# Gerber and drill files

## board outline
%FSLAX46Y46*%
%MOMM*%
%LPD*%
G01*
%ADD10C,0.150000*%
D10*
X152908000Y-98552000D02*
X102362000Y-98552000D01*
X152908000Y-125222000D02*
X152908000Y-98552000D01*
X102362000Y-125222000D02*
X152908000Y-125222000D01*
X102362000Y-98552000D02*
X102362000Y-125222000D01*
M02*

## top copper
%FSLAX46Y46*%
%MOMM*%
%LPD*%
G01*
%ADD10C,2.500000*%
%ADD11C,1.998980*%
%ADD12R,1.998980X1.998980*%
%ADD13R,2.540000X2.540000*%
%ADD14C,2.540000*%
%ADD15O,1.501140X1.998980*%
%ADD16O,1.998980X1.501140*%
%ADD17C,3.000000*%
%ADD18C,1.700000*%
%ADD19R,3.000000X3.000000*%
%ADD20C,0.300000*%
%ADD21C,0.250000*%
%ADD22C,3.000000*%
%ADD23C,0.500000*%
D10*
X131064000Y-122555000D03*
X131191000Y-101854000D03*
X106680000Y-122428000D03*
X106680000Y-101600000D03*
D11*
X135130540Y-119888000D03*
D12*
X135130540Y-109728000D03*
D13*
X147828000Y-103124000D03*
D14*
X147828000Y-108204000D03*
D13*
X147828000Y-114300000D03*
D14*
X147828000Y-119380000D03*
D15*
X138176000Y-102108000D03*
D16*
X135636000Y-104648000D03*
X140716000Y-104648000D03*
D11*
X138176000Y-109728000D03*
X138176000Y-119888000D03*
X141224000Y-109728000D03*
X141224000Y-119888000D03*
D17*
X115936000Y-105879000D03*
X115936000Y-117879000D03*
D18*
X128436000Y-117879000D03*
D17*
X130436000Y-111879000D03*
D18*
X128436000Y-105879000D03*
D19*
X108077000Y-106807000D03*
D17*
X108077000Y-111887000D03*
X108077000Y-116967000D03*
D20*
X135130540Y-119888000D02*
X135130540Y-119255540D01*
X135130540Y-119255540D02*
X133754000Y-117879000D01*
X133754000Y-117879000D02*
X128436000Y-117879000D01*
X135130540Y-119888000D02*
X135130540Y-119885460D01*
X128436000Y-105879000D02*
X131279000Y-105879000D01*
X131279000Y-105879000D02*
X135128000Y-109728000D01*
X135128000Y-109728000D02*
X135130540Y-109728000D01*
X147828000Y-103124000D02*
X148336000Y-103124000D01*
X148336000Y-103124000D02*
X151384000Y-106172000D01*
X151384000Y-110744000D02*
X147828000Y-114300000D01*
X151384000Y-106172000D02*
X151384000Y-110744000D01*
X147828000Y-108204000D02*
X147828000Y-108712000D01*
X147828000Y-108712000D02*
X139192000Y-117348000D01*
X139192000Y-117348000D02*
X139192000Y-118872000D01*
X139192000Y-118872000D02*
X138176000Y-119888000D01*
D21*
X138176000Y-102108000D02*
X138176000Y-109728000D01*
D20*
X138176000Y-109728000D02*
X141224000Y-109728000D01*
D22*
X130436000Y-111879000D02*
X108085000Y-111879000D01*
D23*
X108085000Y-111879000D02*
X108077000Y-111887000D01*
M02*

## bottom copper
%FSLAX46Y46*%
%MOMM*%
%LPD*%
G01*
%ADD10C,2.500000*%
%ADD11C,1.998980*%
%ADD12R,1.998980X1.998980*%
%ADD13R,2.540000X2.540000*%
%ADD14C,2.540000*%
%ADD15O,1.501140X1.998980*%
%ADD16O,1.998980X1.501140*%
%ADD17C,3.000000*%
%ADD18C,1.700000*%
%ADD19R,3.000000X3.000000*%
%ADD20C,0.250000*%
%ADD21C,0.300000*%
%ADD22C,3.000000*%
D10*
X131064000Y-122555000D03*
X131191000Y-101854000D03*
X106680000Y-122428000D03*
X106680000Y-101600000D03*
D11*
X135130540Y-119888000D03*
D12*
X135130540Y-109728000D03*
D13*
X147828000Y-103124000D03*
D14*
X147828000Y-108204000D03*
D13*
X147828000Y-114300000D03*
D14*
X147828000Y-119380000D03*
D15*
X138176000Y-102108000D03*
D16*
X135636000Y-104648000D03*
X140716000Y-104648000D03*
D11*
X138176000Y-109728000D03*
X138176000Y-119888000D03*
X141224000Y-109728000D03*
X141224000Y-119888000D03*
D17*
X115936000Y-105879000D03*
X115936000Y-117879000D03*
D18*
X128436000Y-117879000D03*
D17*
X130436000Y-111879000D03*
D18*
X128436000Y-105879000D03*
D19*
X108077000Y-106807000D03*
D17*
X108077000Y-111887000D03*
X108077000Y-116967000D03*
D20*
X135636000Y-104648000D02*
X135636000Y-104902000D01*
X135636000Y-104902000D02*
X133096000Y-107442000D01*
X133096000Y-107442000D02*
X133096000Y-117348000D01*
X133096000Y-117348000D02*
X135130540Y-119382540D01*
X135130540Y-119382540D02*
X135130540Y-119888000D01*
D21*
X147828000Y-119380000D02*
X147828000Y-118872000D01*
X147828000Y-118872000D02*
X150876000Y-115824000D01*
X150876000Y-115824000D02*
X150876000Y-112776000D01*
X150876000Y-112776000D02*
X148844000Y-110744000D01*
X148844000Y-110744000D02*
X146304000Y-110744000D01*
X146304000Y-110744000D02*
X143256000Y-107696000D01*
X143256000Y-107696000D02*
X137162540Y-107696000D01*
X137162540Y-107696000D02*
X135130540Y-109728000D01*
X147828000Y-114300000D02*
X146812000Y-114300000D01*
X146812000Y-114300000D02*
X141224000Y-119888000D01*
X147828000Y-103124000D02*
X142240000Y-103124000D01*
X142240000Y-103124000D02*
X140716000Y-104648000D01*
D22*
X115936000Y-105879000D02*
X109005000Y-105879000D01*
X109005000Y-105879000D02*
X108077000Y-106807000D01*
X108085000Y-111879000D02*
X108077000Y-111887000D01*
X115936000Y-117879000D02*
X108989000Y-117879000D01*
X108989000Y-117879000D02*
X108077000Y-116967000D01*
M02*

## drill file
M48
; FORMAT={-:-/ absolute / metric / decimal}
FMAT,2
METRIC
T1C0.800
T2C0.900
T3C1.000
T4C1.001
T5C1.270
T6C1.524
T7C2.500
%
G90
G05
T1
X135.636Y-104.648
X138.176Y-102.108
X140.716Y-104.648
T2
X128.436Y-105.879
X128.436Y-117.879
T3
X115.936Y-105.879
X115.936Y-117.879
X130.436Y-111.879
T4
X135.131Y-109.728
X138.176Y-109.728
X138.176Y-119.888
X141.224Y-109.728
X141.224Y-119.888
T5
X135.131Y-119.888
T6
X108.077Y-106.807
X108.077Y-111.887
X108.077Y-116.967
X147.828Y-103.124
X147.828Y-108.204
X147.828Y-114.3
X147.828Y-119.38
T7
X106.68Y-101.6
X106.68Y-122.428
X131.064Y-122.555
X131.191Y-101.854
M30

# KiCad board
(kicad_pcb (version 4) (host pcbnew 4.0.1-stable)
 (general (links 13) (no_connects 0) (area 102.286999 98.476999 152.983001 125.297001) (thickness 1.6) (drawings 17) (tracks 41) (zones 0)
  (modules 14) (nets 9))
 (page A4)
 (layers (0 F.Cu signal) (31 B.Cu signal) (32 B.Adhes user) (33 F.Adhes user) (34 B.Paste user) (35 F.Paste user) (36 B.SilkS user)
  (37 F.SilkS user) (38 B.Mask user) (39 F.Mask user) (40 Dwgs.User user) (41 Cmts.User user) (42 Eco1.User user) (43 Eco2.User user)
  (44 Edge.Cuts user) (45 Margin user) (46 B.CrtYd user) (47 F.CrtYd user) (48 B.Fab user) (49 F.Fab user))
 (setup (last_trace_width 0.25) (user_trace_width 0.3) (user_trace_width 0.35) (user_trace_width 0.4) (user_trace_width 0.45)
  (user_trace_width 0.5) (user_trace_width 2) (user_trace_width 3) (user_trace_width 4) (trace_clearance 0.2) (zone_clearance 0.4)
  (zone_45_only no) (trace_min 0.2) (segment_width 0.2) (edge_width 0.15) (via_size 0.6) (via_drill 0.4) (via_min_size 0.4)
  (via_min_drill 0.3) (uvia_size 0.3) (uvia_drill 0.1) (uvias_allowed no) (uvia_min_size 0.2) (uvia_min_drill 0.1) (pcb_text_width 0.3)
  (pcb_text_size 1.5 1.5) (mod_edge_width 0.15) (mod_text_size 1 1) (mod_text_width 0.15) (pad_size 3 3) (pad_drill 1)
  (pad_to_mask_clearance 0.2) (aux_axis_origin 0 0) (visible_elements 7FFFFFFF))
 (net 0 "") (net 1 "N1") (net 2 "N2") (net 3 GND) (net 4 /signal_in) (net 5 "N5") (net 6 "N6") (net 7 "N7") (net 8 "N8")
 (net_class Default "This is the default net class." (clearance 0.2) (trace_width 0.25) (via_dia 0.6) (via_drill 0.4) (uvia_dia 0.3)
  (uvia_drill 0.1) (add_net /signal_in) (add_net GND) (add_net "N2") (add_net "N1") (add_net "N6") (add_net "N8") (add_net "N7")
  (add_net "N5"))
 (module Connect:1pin (layer F.Cu) (at 131.064 122.555)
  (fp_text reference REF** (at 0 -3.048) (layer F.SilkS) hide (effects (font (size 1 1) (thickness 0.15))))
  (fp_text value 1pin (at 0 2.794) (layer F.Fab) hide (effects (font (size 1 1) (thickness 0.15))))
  (pad 1 thru_hole circle (at 0 0) (size 2.5 2.5) (drill 2.5) (layers *.Cu *.Mask)))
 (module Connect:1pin (layer F.Cu) (at 131.191 101.854)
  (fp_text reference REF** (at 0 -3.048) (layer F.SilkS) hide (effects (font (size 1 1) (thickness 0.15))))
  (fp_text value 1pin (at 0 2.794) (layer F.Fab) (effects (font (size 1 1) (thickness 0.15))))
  (pad 1 thru_hole circle (at 0 0) (size 2.5 2.5) (drill 2.5) (layers *.Cu *.Mask)))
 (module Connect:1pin (layer F.Cu) (at 106.68 122.428)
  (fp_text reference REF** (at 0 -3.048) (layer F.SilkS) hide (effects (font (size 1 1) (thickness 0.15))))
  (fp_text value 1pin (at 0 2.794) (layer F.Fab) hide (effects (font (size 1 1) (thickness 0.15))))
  (pad 1 thru_hole circle (at 0 0) (size 2.5 2.5) (drill 2.5) (layers *.Cu *.Mask)))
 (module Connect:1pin (layer F.Cu) (at 106.68 101.6)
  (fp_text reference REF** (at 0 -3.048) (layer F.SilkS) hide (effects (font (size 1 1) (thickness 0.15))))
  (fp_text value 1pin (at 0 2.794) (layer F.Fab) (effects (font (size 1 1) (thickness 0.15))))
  (pad 1 thru_hole circle (at 0 0) (size 2.5 2.5) (drill 2.5) (layers *.Cu *.Mask)))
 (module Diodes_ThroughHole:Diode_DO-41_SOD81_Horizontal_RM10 (layer F.Cu) (at 135.128 109.728 270)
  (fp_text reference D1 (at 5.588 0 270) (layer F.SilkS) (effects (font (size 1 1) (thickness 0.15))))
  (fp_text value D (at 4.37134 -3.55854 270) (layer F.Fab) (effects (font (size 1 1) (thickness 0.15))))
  (pad 2 thru_hole circle (at 10.16 -0.00254 90) (size 1.99898 1.99898) (drill 1.27) (layers *.Cu *.Mask F.SilkS) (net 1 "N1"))
  (pad 1 thru_hole rect (at 0 -0.00254 90) (size 1.99898 1.99898) (drill 1.00076) (layers *.Cu *.Mask F.SilkS) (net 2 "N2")))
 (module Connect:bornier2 (layer F.Cu) (at 147.828 105.664 270)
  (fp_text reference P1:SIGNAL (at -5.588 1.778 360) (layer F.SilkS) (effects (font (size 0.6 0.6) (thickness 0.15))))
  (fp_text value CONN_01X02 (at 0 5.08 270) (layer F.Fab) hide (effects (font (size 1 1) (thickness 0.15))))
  (pad 1 thru_hole rect (at -2.54 0 270) (size 2.54 2.54) (drill 1.524) (layers *.Cu *.Mask F.SilkS) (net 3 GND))
  (pad 2 thru_hole circle (at 2.54 0 270) (size 2.54 2.54) (drill 1.524) (layers *.Cu *.Mask F.SilkS) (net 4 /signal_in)))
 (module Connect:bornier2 (layer F.Cu) (at 147.828 116.84 270)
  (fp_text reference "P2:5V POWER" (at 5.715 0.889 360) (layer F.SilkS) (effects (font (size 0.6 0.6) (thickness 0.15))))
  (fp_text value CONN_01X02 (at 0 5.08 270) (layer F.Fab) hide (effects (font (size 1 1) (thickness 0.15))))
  (pad 1 thru_hole rect (at -2.54 0 270) (size 2.54 2.54) (drill 1.524) (layers *.Cu *.Mask F.SilkS) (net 3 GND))
  (pad 2 thru_hole circle (at 2.54 0 270) (size 2.54 2.54) (drill 1.524) (layers *.Cu *.Mask F.SilkS) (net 2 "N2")))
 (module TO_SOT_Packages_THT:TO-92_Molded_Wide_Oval (layer F.Cu) (at 135.636 104.648)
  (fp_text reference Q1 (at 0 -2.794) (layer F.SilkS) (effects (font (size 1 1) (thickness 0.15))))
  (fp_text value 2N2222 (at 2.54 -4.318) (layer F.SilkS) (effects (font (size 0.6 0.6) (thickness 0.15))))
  (pad 1 thru_hole oval (at 2.54 -2.54 90) (size 1.99898 1.50114) (drill 0.8) (layers *.Cu *.Mask F.SilkS) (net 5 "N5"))
  (pad 2 thru_hole oval (at 0 0 90) (size 1.50114 1.99898) (drill 0.8) (layers *.Cu *.Mask F.SilkS) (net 1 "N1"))
  (pad 3 thru_hole oval (at 5.08 0 90) (size 1.50114 1.99898) (drill 0.8) (layers *.Cu *.Mask F.SilkS) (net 3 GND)))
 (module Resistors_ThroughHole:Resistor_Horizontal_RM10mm (layer F.Cu) (at 138.176 114.808 270)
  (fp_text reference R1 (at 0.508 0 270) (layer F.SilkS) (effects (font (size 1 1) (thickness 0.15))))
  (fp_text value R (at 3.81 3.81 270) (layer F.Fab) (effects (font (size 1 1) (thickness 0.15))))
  (pad 1 thru_hole circle (at -5.08 0 270) (size 1.99898 1.99898) (drill 1.00076) (layers *.Cu *.SilkS *.Mask) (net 5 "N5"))
  (pad 2 thru_hole circle (at 5.08 0 270) (size 1.99898 1.99898) (drill 1.00076) (layers *.Cu *.SilkS *.Mask) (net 4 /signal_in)))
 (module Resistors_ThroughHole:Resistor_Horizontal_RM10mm (layer F.Cu) (at 141.224 114.808 270)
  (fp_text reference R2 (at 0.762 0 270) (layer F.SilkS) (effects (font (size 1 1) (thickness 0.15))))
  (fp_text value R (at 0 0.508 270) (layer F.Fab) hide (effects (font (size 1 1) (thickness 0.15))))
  (pad 1 thru_hole circle (at -5.08 0 270) (size 1.99898 1.99898) (drill 1.00076) (layers *.Cu *.SilkS *.Mask) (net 5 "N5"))
  (pad 2 thru_hole circle (at 5.08 0 270) (size 1.99898 1.99898) (drill 1.00076) (layers *.Cu *.SilkS *.Mask) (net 3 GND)))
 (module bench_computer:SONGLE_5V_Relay (layer F.Cu) (at 122.936 111.379)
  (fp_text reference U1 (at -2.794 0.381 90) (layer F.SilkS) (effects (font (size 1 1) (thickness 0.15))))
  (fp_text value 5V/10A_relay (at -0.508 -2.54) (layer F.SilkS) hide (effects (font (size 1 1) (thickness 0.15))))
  (pad 4 thru_hole circle (at -7 -5.5) (size 3 3) (drill 1) (layers *.Cu *.Mask F.SilkS) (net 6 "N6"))
  (pad 5 thru_hole circle (at -7 6.5) (size 3 3) (drill 1) (layers *.Cu *.Mask F.SilkS) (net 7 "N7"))
  (pad 2 thru_hole circle (at 5.5 6.5) (size 1.7 1.7) (drill 0.9) (layers *.Cu *.Mask F.SilkS) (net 1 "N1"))
  (pad 3 thru_hole circle (at 7.5 0.5) (size 3 3) (drill 1) (layers *.Cu *.Mask F.SilkS) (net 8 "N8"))
  (pad 1 thru_hole circle (at 5.5 -5.5) (size 1.7 1.7) (drill 0.9) (layers *.Cu *.Mask F.SilkS) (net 2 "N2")))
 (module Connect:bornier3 (layer F.Cu) (at 108.077 111.887 270)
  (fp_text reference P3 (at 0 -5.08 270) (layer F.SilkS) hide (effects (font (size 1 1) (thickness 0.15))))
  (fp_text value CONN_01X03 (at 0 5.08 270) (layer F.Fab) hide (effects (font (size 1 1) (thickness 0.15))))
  (pad 1 thru_hole rect (at -5.08 0 270) (size 3 3) (drill 1.524) (layers *.Cu *.Mask F.SilkS) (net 6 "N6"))
  (pad 2 thru_hole circle (at 0 0 270) (size 3 3) (drill 1.524) (layers *.Cu *.Mask F.SilkS) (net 8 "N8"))
  (pad 3 thru_hole circle (at 5.08 0 270) (size 3 3) (drill 1.524) (layers *.Cu *.Mask F.SilkS) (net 7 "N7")))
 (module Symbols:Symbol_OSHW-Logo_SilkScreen (layer B.Cu) (at 122.428 111.125 180)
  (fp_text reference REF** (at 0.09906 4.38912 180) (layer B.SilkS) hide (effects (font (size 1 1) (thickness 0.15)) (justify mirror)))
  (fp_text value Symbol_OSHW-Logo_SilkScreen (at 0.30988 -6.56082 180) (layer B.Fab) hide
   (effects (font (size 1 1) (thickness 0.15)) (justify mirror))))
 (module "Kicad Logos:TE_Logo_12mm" (layer F.Cu) (at 118.364 101.219)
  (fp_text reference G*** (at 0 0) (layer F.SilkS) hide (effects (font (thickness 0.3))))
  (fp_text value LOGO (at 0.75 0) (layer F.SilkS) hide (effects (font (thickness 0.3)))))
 (gr_line (start 152.908 98.552) (end 102.362 98.552) (angle 90) (layer Edge.Cuts) (width 0.15))
 (gr_line (start 152.908 125.222) (end 152.908 98.552) (angle 90) (layer Edge.Cuts) (width 0.15))
 (gr_line (start 102.362 125.222) (end 152.908 125.222) (angle 90) (layer Edge.Cuts) (width 0.15))
 (gr_line (start 102.362 98.552) (end 102.362 125.222) (angle 90) (layer Edge.Cuts) (width 0.15))
 (segment (start 135.636 104.648) (end 135.636 104.902) (width 0.25) (layer B.Cu) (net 1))
 (segment (start 135.636 104.902) (end 133.096 107.442) (width 0.25) (layer B.Cu) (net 1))
 (segment (start 133.096 107.442) (end 133.096 117.348) (width 0.25) (layer B.Cu) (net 1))
 (segment (start 133.096 117.348) (end 135.13054 119.38254) (width 0.25) (layer B.Cu) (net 1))
 (segment (start 135.13054 119.38254) (end 135.13054 119.888) (width 0.25) (layer B.Cu) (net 1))
 (segment (start 135.13054 119.888) (end 135.13054 119.25554) (width 0.3) (layer F.Cu) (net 1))
 (segment (start 135.13054 119.25554) (end 133.754 117.879) (width 0.3) (layer F.Cu) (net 1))
 (segment (start 133.754 117.879) (end 128.436 117.879) (width 0.3) (layer F.Cu) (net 1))
 (segment (start 135.13054 119.888) (end 135.13054 119.88546) (width 0.3) (layer F.Cu) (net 1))
 (segment (start 147.828 119.38) (end 147.828 118.872) (width 0.3) (layer B.Cu) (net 2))
 (segment (start 147.828 118.872) (end 150.876 115.824) (width 0.3) (layer B.Cu) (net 2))
 (segment (start 150.876 115.824) (end 150.876 112.776) (width 0.3) (layer B.Cu) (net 2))
 (segment (start 150.876 112.776) (end 148.844 110.744) (width 0.3) (layer B.Cu) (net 2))
 (segment (start 148.844 110.744) (end 146.304 110.744) (width 0.3) (layer B.Cu) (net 2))
 (segment (start 146.304 110.744) (end 143.256 107.696) (width 0.3) (layer B.Cu) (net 2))
 (segment (start 143.256 107.696) (end 137.16254 107.696) (width 0.3) (layer B.Cu) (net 2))
 (segment (start 137.16254 107.696) (end 135.13054 109.728) (width 0.3) (layer B.Cu) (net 2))
 (segment (start 128.436 105.879) (end 131.279 105.879) (width 0.3) (layer F.Cu) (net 2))
 (segment (start 131.279 105.879) (end 135.128 109.728) (width 0.3) (layer F.Cu) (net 2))
 (segment (start 135.128 109.728) (end 135.13054 109.728) (width 0.3) (layer F.Cu) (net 2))
 (segment (start 147.828 103.124) (end 148.336 103.124) (width 0.3) (layer F.Cu) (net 3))
 (segment (start 148.336 103.124) (end 151.384 106.172) (width 0.3) (layer F.Cu) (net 3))
 (segment (start 151.384 110.744) (end 147.828 114.3) (width 0.3) (layer F.Cu) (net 3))
 (segment (start 151.384 106.172) (end 151.384 110.744) (width 0.3) (layer F.Cu) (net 3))
 (segment (start 147.828 114.3) (end 146.812 114.3) (width 0.3) (layer B.Cu) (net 3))
 (segment (start 146.812 114.3) (end 141.224 119.888) (width 0.3) (layer B.Cu) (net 3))
 (segment (start 147.828 103.124) (end 142.24 103.124) (width 0.3) (layer B.Cu) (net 3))
 (segment (start 142.24 103.124) (end 140.716 104.648) (width 0.3) (layer B.Cu) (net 3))
 (segment (start 147.828 108.204) (end 147.828 108.712) (width 0.3) (layer F.Cu) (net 4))
 (segment (start 147.828 108.712) (end 139.192 117.348) (width 0.3) (layer F.Cu) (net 4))
 (segment (start 139.192 117.348) (end 139.192 118.872) (width 0.3) (layer F.Cu) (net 4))
 (segment (start 139.192 118.872) (end 138.176 119.888) (width 0.3) (layer F.Cu) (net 4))
 (segment (start 138.176 102.108) (end 138.176 109.728) (width 0.25) (layer F.Cu) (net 5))
 (segment (start 138.176 109.728) (end 141.224 109.728) (width 0.3) (layer F.Cu) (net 5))
 (segment (start 115.936 105.879) (end 109.005 105.879) (width 3) (layer B.Cu) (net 6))
 (segment (start 109.005 105.879) (end 108.077 106.807) (width 3) (layer B.Cu) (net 6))
 (segment (start 130.436 111.879) (end 108.085 111.879) (width 3) (layer F.Cu) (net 8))
 (segment (start 108.085 111.879) (end 108.077 111.887) (width 0.5) (layer F.Cu) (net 8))
 (segment (start 108.085 111.879) (end 108.077 111.887) (width 3) (layer B.Cu) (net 8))
 (segment (start 115.936 117.879) (end 108.989 117.879) (width 3) (layer B.Cu) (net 7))
 (segment (start 108.989 117.879) (end 108.077 116.967) (width 3) (layer B.Cu) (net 7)))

